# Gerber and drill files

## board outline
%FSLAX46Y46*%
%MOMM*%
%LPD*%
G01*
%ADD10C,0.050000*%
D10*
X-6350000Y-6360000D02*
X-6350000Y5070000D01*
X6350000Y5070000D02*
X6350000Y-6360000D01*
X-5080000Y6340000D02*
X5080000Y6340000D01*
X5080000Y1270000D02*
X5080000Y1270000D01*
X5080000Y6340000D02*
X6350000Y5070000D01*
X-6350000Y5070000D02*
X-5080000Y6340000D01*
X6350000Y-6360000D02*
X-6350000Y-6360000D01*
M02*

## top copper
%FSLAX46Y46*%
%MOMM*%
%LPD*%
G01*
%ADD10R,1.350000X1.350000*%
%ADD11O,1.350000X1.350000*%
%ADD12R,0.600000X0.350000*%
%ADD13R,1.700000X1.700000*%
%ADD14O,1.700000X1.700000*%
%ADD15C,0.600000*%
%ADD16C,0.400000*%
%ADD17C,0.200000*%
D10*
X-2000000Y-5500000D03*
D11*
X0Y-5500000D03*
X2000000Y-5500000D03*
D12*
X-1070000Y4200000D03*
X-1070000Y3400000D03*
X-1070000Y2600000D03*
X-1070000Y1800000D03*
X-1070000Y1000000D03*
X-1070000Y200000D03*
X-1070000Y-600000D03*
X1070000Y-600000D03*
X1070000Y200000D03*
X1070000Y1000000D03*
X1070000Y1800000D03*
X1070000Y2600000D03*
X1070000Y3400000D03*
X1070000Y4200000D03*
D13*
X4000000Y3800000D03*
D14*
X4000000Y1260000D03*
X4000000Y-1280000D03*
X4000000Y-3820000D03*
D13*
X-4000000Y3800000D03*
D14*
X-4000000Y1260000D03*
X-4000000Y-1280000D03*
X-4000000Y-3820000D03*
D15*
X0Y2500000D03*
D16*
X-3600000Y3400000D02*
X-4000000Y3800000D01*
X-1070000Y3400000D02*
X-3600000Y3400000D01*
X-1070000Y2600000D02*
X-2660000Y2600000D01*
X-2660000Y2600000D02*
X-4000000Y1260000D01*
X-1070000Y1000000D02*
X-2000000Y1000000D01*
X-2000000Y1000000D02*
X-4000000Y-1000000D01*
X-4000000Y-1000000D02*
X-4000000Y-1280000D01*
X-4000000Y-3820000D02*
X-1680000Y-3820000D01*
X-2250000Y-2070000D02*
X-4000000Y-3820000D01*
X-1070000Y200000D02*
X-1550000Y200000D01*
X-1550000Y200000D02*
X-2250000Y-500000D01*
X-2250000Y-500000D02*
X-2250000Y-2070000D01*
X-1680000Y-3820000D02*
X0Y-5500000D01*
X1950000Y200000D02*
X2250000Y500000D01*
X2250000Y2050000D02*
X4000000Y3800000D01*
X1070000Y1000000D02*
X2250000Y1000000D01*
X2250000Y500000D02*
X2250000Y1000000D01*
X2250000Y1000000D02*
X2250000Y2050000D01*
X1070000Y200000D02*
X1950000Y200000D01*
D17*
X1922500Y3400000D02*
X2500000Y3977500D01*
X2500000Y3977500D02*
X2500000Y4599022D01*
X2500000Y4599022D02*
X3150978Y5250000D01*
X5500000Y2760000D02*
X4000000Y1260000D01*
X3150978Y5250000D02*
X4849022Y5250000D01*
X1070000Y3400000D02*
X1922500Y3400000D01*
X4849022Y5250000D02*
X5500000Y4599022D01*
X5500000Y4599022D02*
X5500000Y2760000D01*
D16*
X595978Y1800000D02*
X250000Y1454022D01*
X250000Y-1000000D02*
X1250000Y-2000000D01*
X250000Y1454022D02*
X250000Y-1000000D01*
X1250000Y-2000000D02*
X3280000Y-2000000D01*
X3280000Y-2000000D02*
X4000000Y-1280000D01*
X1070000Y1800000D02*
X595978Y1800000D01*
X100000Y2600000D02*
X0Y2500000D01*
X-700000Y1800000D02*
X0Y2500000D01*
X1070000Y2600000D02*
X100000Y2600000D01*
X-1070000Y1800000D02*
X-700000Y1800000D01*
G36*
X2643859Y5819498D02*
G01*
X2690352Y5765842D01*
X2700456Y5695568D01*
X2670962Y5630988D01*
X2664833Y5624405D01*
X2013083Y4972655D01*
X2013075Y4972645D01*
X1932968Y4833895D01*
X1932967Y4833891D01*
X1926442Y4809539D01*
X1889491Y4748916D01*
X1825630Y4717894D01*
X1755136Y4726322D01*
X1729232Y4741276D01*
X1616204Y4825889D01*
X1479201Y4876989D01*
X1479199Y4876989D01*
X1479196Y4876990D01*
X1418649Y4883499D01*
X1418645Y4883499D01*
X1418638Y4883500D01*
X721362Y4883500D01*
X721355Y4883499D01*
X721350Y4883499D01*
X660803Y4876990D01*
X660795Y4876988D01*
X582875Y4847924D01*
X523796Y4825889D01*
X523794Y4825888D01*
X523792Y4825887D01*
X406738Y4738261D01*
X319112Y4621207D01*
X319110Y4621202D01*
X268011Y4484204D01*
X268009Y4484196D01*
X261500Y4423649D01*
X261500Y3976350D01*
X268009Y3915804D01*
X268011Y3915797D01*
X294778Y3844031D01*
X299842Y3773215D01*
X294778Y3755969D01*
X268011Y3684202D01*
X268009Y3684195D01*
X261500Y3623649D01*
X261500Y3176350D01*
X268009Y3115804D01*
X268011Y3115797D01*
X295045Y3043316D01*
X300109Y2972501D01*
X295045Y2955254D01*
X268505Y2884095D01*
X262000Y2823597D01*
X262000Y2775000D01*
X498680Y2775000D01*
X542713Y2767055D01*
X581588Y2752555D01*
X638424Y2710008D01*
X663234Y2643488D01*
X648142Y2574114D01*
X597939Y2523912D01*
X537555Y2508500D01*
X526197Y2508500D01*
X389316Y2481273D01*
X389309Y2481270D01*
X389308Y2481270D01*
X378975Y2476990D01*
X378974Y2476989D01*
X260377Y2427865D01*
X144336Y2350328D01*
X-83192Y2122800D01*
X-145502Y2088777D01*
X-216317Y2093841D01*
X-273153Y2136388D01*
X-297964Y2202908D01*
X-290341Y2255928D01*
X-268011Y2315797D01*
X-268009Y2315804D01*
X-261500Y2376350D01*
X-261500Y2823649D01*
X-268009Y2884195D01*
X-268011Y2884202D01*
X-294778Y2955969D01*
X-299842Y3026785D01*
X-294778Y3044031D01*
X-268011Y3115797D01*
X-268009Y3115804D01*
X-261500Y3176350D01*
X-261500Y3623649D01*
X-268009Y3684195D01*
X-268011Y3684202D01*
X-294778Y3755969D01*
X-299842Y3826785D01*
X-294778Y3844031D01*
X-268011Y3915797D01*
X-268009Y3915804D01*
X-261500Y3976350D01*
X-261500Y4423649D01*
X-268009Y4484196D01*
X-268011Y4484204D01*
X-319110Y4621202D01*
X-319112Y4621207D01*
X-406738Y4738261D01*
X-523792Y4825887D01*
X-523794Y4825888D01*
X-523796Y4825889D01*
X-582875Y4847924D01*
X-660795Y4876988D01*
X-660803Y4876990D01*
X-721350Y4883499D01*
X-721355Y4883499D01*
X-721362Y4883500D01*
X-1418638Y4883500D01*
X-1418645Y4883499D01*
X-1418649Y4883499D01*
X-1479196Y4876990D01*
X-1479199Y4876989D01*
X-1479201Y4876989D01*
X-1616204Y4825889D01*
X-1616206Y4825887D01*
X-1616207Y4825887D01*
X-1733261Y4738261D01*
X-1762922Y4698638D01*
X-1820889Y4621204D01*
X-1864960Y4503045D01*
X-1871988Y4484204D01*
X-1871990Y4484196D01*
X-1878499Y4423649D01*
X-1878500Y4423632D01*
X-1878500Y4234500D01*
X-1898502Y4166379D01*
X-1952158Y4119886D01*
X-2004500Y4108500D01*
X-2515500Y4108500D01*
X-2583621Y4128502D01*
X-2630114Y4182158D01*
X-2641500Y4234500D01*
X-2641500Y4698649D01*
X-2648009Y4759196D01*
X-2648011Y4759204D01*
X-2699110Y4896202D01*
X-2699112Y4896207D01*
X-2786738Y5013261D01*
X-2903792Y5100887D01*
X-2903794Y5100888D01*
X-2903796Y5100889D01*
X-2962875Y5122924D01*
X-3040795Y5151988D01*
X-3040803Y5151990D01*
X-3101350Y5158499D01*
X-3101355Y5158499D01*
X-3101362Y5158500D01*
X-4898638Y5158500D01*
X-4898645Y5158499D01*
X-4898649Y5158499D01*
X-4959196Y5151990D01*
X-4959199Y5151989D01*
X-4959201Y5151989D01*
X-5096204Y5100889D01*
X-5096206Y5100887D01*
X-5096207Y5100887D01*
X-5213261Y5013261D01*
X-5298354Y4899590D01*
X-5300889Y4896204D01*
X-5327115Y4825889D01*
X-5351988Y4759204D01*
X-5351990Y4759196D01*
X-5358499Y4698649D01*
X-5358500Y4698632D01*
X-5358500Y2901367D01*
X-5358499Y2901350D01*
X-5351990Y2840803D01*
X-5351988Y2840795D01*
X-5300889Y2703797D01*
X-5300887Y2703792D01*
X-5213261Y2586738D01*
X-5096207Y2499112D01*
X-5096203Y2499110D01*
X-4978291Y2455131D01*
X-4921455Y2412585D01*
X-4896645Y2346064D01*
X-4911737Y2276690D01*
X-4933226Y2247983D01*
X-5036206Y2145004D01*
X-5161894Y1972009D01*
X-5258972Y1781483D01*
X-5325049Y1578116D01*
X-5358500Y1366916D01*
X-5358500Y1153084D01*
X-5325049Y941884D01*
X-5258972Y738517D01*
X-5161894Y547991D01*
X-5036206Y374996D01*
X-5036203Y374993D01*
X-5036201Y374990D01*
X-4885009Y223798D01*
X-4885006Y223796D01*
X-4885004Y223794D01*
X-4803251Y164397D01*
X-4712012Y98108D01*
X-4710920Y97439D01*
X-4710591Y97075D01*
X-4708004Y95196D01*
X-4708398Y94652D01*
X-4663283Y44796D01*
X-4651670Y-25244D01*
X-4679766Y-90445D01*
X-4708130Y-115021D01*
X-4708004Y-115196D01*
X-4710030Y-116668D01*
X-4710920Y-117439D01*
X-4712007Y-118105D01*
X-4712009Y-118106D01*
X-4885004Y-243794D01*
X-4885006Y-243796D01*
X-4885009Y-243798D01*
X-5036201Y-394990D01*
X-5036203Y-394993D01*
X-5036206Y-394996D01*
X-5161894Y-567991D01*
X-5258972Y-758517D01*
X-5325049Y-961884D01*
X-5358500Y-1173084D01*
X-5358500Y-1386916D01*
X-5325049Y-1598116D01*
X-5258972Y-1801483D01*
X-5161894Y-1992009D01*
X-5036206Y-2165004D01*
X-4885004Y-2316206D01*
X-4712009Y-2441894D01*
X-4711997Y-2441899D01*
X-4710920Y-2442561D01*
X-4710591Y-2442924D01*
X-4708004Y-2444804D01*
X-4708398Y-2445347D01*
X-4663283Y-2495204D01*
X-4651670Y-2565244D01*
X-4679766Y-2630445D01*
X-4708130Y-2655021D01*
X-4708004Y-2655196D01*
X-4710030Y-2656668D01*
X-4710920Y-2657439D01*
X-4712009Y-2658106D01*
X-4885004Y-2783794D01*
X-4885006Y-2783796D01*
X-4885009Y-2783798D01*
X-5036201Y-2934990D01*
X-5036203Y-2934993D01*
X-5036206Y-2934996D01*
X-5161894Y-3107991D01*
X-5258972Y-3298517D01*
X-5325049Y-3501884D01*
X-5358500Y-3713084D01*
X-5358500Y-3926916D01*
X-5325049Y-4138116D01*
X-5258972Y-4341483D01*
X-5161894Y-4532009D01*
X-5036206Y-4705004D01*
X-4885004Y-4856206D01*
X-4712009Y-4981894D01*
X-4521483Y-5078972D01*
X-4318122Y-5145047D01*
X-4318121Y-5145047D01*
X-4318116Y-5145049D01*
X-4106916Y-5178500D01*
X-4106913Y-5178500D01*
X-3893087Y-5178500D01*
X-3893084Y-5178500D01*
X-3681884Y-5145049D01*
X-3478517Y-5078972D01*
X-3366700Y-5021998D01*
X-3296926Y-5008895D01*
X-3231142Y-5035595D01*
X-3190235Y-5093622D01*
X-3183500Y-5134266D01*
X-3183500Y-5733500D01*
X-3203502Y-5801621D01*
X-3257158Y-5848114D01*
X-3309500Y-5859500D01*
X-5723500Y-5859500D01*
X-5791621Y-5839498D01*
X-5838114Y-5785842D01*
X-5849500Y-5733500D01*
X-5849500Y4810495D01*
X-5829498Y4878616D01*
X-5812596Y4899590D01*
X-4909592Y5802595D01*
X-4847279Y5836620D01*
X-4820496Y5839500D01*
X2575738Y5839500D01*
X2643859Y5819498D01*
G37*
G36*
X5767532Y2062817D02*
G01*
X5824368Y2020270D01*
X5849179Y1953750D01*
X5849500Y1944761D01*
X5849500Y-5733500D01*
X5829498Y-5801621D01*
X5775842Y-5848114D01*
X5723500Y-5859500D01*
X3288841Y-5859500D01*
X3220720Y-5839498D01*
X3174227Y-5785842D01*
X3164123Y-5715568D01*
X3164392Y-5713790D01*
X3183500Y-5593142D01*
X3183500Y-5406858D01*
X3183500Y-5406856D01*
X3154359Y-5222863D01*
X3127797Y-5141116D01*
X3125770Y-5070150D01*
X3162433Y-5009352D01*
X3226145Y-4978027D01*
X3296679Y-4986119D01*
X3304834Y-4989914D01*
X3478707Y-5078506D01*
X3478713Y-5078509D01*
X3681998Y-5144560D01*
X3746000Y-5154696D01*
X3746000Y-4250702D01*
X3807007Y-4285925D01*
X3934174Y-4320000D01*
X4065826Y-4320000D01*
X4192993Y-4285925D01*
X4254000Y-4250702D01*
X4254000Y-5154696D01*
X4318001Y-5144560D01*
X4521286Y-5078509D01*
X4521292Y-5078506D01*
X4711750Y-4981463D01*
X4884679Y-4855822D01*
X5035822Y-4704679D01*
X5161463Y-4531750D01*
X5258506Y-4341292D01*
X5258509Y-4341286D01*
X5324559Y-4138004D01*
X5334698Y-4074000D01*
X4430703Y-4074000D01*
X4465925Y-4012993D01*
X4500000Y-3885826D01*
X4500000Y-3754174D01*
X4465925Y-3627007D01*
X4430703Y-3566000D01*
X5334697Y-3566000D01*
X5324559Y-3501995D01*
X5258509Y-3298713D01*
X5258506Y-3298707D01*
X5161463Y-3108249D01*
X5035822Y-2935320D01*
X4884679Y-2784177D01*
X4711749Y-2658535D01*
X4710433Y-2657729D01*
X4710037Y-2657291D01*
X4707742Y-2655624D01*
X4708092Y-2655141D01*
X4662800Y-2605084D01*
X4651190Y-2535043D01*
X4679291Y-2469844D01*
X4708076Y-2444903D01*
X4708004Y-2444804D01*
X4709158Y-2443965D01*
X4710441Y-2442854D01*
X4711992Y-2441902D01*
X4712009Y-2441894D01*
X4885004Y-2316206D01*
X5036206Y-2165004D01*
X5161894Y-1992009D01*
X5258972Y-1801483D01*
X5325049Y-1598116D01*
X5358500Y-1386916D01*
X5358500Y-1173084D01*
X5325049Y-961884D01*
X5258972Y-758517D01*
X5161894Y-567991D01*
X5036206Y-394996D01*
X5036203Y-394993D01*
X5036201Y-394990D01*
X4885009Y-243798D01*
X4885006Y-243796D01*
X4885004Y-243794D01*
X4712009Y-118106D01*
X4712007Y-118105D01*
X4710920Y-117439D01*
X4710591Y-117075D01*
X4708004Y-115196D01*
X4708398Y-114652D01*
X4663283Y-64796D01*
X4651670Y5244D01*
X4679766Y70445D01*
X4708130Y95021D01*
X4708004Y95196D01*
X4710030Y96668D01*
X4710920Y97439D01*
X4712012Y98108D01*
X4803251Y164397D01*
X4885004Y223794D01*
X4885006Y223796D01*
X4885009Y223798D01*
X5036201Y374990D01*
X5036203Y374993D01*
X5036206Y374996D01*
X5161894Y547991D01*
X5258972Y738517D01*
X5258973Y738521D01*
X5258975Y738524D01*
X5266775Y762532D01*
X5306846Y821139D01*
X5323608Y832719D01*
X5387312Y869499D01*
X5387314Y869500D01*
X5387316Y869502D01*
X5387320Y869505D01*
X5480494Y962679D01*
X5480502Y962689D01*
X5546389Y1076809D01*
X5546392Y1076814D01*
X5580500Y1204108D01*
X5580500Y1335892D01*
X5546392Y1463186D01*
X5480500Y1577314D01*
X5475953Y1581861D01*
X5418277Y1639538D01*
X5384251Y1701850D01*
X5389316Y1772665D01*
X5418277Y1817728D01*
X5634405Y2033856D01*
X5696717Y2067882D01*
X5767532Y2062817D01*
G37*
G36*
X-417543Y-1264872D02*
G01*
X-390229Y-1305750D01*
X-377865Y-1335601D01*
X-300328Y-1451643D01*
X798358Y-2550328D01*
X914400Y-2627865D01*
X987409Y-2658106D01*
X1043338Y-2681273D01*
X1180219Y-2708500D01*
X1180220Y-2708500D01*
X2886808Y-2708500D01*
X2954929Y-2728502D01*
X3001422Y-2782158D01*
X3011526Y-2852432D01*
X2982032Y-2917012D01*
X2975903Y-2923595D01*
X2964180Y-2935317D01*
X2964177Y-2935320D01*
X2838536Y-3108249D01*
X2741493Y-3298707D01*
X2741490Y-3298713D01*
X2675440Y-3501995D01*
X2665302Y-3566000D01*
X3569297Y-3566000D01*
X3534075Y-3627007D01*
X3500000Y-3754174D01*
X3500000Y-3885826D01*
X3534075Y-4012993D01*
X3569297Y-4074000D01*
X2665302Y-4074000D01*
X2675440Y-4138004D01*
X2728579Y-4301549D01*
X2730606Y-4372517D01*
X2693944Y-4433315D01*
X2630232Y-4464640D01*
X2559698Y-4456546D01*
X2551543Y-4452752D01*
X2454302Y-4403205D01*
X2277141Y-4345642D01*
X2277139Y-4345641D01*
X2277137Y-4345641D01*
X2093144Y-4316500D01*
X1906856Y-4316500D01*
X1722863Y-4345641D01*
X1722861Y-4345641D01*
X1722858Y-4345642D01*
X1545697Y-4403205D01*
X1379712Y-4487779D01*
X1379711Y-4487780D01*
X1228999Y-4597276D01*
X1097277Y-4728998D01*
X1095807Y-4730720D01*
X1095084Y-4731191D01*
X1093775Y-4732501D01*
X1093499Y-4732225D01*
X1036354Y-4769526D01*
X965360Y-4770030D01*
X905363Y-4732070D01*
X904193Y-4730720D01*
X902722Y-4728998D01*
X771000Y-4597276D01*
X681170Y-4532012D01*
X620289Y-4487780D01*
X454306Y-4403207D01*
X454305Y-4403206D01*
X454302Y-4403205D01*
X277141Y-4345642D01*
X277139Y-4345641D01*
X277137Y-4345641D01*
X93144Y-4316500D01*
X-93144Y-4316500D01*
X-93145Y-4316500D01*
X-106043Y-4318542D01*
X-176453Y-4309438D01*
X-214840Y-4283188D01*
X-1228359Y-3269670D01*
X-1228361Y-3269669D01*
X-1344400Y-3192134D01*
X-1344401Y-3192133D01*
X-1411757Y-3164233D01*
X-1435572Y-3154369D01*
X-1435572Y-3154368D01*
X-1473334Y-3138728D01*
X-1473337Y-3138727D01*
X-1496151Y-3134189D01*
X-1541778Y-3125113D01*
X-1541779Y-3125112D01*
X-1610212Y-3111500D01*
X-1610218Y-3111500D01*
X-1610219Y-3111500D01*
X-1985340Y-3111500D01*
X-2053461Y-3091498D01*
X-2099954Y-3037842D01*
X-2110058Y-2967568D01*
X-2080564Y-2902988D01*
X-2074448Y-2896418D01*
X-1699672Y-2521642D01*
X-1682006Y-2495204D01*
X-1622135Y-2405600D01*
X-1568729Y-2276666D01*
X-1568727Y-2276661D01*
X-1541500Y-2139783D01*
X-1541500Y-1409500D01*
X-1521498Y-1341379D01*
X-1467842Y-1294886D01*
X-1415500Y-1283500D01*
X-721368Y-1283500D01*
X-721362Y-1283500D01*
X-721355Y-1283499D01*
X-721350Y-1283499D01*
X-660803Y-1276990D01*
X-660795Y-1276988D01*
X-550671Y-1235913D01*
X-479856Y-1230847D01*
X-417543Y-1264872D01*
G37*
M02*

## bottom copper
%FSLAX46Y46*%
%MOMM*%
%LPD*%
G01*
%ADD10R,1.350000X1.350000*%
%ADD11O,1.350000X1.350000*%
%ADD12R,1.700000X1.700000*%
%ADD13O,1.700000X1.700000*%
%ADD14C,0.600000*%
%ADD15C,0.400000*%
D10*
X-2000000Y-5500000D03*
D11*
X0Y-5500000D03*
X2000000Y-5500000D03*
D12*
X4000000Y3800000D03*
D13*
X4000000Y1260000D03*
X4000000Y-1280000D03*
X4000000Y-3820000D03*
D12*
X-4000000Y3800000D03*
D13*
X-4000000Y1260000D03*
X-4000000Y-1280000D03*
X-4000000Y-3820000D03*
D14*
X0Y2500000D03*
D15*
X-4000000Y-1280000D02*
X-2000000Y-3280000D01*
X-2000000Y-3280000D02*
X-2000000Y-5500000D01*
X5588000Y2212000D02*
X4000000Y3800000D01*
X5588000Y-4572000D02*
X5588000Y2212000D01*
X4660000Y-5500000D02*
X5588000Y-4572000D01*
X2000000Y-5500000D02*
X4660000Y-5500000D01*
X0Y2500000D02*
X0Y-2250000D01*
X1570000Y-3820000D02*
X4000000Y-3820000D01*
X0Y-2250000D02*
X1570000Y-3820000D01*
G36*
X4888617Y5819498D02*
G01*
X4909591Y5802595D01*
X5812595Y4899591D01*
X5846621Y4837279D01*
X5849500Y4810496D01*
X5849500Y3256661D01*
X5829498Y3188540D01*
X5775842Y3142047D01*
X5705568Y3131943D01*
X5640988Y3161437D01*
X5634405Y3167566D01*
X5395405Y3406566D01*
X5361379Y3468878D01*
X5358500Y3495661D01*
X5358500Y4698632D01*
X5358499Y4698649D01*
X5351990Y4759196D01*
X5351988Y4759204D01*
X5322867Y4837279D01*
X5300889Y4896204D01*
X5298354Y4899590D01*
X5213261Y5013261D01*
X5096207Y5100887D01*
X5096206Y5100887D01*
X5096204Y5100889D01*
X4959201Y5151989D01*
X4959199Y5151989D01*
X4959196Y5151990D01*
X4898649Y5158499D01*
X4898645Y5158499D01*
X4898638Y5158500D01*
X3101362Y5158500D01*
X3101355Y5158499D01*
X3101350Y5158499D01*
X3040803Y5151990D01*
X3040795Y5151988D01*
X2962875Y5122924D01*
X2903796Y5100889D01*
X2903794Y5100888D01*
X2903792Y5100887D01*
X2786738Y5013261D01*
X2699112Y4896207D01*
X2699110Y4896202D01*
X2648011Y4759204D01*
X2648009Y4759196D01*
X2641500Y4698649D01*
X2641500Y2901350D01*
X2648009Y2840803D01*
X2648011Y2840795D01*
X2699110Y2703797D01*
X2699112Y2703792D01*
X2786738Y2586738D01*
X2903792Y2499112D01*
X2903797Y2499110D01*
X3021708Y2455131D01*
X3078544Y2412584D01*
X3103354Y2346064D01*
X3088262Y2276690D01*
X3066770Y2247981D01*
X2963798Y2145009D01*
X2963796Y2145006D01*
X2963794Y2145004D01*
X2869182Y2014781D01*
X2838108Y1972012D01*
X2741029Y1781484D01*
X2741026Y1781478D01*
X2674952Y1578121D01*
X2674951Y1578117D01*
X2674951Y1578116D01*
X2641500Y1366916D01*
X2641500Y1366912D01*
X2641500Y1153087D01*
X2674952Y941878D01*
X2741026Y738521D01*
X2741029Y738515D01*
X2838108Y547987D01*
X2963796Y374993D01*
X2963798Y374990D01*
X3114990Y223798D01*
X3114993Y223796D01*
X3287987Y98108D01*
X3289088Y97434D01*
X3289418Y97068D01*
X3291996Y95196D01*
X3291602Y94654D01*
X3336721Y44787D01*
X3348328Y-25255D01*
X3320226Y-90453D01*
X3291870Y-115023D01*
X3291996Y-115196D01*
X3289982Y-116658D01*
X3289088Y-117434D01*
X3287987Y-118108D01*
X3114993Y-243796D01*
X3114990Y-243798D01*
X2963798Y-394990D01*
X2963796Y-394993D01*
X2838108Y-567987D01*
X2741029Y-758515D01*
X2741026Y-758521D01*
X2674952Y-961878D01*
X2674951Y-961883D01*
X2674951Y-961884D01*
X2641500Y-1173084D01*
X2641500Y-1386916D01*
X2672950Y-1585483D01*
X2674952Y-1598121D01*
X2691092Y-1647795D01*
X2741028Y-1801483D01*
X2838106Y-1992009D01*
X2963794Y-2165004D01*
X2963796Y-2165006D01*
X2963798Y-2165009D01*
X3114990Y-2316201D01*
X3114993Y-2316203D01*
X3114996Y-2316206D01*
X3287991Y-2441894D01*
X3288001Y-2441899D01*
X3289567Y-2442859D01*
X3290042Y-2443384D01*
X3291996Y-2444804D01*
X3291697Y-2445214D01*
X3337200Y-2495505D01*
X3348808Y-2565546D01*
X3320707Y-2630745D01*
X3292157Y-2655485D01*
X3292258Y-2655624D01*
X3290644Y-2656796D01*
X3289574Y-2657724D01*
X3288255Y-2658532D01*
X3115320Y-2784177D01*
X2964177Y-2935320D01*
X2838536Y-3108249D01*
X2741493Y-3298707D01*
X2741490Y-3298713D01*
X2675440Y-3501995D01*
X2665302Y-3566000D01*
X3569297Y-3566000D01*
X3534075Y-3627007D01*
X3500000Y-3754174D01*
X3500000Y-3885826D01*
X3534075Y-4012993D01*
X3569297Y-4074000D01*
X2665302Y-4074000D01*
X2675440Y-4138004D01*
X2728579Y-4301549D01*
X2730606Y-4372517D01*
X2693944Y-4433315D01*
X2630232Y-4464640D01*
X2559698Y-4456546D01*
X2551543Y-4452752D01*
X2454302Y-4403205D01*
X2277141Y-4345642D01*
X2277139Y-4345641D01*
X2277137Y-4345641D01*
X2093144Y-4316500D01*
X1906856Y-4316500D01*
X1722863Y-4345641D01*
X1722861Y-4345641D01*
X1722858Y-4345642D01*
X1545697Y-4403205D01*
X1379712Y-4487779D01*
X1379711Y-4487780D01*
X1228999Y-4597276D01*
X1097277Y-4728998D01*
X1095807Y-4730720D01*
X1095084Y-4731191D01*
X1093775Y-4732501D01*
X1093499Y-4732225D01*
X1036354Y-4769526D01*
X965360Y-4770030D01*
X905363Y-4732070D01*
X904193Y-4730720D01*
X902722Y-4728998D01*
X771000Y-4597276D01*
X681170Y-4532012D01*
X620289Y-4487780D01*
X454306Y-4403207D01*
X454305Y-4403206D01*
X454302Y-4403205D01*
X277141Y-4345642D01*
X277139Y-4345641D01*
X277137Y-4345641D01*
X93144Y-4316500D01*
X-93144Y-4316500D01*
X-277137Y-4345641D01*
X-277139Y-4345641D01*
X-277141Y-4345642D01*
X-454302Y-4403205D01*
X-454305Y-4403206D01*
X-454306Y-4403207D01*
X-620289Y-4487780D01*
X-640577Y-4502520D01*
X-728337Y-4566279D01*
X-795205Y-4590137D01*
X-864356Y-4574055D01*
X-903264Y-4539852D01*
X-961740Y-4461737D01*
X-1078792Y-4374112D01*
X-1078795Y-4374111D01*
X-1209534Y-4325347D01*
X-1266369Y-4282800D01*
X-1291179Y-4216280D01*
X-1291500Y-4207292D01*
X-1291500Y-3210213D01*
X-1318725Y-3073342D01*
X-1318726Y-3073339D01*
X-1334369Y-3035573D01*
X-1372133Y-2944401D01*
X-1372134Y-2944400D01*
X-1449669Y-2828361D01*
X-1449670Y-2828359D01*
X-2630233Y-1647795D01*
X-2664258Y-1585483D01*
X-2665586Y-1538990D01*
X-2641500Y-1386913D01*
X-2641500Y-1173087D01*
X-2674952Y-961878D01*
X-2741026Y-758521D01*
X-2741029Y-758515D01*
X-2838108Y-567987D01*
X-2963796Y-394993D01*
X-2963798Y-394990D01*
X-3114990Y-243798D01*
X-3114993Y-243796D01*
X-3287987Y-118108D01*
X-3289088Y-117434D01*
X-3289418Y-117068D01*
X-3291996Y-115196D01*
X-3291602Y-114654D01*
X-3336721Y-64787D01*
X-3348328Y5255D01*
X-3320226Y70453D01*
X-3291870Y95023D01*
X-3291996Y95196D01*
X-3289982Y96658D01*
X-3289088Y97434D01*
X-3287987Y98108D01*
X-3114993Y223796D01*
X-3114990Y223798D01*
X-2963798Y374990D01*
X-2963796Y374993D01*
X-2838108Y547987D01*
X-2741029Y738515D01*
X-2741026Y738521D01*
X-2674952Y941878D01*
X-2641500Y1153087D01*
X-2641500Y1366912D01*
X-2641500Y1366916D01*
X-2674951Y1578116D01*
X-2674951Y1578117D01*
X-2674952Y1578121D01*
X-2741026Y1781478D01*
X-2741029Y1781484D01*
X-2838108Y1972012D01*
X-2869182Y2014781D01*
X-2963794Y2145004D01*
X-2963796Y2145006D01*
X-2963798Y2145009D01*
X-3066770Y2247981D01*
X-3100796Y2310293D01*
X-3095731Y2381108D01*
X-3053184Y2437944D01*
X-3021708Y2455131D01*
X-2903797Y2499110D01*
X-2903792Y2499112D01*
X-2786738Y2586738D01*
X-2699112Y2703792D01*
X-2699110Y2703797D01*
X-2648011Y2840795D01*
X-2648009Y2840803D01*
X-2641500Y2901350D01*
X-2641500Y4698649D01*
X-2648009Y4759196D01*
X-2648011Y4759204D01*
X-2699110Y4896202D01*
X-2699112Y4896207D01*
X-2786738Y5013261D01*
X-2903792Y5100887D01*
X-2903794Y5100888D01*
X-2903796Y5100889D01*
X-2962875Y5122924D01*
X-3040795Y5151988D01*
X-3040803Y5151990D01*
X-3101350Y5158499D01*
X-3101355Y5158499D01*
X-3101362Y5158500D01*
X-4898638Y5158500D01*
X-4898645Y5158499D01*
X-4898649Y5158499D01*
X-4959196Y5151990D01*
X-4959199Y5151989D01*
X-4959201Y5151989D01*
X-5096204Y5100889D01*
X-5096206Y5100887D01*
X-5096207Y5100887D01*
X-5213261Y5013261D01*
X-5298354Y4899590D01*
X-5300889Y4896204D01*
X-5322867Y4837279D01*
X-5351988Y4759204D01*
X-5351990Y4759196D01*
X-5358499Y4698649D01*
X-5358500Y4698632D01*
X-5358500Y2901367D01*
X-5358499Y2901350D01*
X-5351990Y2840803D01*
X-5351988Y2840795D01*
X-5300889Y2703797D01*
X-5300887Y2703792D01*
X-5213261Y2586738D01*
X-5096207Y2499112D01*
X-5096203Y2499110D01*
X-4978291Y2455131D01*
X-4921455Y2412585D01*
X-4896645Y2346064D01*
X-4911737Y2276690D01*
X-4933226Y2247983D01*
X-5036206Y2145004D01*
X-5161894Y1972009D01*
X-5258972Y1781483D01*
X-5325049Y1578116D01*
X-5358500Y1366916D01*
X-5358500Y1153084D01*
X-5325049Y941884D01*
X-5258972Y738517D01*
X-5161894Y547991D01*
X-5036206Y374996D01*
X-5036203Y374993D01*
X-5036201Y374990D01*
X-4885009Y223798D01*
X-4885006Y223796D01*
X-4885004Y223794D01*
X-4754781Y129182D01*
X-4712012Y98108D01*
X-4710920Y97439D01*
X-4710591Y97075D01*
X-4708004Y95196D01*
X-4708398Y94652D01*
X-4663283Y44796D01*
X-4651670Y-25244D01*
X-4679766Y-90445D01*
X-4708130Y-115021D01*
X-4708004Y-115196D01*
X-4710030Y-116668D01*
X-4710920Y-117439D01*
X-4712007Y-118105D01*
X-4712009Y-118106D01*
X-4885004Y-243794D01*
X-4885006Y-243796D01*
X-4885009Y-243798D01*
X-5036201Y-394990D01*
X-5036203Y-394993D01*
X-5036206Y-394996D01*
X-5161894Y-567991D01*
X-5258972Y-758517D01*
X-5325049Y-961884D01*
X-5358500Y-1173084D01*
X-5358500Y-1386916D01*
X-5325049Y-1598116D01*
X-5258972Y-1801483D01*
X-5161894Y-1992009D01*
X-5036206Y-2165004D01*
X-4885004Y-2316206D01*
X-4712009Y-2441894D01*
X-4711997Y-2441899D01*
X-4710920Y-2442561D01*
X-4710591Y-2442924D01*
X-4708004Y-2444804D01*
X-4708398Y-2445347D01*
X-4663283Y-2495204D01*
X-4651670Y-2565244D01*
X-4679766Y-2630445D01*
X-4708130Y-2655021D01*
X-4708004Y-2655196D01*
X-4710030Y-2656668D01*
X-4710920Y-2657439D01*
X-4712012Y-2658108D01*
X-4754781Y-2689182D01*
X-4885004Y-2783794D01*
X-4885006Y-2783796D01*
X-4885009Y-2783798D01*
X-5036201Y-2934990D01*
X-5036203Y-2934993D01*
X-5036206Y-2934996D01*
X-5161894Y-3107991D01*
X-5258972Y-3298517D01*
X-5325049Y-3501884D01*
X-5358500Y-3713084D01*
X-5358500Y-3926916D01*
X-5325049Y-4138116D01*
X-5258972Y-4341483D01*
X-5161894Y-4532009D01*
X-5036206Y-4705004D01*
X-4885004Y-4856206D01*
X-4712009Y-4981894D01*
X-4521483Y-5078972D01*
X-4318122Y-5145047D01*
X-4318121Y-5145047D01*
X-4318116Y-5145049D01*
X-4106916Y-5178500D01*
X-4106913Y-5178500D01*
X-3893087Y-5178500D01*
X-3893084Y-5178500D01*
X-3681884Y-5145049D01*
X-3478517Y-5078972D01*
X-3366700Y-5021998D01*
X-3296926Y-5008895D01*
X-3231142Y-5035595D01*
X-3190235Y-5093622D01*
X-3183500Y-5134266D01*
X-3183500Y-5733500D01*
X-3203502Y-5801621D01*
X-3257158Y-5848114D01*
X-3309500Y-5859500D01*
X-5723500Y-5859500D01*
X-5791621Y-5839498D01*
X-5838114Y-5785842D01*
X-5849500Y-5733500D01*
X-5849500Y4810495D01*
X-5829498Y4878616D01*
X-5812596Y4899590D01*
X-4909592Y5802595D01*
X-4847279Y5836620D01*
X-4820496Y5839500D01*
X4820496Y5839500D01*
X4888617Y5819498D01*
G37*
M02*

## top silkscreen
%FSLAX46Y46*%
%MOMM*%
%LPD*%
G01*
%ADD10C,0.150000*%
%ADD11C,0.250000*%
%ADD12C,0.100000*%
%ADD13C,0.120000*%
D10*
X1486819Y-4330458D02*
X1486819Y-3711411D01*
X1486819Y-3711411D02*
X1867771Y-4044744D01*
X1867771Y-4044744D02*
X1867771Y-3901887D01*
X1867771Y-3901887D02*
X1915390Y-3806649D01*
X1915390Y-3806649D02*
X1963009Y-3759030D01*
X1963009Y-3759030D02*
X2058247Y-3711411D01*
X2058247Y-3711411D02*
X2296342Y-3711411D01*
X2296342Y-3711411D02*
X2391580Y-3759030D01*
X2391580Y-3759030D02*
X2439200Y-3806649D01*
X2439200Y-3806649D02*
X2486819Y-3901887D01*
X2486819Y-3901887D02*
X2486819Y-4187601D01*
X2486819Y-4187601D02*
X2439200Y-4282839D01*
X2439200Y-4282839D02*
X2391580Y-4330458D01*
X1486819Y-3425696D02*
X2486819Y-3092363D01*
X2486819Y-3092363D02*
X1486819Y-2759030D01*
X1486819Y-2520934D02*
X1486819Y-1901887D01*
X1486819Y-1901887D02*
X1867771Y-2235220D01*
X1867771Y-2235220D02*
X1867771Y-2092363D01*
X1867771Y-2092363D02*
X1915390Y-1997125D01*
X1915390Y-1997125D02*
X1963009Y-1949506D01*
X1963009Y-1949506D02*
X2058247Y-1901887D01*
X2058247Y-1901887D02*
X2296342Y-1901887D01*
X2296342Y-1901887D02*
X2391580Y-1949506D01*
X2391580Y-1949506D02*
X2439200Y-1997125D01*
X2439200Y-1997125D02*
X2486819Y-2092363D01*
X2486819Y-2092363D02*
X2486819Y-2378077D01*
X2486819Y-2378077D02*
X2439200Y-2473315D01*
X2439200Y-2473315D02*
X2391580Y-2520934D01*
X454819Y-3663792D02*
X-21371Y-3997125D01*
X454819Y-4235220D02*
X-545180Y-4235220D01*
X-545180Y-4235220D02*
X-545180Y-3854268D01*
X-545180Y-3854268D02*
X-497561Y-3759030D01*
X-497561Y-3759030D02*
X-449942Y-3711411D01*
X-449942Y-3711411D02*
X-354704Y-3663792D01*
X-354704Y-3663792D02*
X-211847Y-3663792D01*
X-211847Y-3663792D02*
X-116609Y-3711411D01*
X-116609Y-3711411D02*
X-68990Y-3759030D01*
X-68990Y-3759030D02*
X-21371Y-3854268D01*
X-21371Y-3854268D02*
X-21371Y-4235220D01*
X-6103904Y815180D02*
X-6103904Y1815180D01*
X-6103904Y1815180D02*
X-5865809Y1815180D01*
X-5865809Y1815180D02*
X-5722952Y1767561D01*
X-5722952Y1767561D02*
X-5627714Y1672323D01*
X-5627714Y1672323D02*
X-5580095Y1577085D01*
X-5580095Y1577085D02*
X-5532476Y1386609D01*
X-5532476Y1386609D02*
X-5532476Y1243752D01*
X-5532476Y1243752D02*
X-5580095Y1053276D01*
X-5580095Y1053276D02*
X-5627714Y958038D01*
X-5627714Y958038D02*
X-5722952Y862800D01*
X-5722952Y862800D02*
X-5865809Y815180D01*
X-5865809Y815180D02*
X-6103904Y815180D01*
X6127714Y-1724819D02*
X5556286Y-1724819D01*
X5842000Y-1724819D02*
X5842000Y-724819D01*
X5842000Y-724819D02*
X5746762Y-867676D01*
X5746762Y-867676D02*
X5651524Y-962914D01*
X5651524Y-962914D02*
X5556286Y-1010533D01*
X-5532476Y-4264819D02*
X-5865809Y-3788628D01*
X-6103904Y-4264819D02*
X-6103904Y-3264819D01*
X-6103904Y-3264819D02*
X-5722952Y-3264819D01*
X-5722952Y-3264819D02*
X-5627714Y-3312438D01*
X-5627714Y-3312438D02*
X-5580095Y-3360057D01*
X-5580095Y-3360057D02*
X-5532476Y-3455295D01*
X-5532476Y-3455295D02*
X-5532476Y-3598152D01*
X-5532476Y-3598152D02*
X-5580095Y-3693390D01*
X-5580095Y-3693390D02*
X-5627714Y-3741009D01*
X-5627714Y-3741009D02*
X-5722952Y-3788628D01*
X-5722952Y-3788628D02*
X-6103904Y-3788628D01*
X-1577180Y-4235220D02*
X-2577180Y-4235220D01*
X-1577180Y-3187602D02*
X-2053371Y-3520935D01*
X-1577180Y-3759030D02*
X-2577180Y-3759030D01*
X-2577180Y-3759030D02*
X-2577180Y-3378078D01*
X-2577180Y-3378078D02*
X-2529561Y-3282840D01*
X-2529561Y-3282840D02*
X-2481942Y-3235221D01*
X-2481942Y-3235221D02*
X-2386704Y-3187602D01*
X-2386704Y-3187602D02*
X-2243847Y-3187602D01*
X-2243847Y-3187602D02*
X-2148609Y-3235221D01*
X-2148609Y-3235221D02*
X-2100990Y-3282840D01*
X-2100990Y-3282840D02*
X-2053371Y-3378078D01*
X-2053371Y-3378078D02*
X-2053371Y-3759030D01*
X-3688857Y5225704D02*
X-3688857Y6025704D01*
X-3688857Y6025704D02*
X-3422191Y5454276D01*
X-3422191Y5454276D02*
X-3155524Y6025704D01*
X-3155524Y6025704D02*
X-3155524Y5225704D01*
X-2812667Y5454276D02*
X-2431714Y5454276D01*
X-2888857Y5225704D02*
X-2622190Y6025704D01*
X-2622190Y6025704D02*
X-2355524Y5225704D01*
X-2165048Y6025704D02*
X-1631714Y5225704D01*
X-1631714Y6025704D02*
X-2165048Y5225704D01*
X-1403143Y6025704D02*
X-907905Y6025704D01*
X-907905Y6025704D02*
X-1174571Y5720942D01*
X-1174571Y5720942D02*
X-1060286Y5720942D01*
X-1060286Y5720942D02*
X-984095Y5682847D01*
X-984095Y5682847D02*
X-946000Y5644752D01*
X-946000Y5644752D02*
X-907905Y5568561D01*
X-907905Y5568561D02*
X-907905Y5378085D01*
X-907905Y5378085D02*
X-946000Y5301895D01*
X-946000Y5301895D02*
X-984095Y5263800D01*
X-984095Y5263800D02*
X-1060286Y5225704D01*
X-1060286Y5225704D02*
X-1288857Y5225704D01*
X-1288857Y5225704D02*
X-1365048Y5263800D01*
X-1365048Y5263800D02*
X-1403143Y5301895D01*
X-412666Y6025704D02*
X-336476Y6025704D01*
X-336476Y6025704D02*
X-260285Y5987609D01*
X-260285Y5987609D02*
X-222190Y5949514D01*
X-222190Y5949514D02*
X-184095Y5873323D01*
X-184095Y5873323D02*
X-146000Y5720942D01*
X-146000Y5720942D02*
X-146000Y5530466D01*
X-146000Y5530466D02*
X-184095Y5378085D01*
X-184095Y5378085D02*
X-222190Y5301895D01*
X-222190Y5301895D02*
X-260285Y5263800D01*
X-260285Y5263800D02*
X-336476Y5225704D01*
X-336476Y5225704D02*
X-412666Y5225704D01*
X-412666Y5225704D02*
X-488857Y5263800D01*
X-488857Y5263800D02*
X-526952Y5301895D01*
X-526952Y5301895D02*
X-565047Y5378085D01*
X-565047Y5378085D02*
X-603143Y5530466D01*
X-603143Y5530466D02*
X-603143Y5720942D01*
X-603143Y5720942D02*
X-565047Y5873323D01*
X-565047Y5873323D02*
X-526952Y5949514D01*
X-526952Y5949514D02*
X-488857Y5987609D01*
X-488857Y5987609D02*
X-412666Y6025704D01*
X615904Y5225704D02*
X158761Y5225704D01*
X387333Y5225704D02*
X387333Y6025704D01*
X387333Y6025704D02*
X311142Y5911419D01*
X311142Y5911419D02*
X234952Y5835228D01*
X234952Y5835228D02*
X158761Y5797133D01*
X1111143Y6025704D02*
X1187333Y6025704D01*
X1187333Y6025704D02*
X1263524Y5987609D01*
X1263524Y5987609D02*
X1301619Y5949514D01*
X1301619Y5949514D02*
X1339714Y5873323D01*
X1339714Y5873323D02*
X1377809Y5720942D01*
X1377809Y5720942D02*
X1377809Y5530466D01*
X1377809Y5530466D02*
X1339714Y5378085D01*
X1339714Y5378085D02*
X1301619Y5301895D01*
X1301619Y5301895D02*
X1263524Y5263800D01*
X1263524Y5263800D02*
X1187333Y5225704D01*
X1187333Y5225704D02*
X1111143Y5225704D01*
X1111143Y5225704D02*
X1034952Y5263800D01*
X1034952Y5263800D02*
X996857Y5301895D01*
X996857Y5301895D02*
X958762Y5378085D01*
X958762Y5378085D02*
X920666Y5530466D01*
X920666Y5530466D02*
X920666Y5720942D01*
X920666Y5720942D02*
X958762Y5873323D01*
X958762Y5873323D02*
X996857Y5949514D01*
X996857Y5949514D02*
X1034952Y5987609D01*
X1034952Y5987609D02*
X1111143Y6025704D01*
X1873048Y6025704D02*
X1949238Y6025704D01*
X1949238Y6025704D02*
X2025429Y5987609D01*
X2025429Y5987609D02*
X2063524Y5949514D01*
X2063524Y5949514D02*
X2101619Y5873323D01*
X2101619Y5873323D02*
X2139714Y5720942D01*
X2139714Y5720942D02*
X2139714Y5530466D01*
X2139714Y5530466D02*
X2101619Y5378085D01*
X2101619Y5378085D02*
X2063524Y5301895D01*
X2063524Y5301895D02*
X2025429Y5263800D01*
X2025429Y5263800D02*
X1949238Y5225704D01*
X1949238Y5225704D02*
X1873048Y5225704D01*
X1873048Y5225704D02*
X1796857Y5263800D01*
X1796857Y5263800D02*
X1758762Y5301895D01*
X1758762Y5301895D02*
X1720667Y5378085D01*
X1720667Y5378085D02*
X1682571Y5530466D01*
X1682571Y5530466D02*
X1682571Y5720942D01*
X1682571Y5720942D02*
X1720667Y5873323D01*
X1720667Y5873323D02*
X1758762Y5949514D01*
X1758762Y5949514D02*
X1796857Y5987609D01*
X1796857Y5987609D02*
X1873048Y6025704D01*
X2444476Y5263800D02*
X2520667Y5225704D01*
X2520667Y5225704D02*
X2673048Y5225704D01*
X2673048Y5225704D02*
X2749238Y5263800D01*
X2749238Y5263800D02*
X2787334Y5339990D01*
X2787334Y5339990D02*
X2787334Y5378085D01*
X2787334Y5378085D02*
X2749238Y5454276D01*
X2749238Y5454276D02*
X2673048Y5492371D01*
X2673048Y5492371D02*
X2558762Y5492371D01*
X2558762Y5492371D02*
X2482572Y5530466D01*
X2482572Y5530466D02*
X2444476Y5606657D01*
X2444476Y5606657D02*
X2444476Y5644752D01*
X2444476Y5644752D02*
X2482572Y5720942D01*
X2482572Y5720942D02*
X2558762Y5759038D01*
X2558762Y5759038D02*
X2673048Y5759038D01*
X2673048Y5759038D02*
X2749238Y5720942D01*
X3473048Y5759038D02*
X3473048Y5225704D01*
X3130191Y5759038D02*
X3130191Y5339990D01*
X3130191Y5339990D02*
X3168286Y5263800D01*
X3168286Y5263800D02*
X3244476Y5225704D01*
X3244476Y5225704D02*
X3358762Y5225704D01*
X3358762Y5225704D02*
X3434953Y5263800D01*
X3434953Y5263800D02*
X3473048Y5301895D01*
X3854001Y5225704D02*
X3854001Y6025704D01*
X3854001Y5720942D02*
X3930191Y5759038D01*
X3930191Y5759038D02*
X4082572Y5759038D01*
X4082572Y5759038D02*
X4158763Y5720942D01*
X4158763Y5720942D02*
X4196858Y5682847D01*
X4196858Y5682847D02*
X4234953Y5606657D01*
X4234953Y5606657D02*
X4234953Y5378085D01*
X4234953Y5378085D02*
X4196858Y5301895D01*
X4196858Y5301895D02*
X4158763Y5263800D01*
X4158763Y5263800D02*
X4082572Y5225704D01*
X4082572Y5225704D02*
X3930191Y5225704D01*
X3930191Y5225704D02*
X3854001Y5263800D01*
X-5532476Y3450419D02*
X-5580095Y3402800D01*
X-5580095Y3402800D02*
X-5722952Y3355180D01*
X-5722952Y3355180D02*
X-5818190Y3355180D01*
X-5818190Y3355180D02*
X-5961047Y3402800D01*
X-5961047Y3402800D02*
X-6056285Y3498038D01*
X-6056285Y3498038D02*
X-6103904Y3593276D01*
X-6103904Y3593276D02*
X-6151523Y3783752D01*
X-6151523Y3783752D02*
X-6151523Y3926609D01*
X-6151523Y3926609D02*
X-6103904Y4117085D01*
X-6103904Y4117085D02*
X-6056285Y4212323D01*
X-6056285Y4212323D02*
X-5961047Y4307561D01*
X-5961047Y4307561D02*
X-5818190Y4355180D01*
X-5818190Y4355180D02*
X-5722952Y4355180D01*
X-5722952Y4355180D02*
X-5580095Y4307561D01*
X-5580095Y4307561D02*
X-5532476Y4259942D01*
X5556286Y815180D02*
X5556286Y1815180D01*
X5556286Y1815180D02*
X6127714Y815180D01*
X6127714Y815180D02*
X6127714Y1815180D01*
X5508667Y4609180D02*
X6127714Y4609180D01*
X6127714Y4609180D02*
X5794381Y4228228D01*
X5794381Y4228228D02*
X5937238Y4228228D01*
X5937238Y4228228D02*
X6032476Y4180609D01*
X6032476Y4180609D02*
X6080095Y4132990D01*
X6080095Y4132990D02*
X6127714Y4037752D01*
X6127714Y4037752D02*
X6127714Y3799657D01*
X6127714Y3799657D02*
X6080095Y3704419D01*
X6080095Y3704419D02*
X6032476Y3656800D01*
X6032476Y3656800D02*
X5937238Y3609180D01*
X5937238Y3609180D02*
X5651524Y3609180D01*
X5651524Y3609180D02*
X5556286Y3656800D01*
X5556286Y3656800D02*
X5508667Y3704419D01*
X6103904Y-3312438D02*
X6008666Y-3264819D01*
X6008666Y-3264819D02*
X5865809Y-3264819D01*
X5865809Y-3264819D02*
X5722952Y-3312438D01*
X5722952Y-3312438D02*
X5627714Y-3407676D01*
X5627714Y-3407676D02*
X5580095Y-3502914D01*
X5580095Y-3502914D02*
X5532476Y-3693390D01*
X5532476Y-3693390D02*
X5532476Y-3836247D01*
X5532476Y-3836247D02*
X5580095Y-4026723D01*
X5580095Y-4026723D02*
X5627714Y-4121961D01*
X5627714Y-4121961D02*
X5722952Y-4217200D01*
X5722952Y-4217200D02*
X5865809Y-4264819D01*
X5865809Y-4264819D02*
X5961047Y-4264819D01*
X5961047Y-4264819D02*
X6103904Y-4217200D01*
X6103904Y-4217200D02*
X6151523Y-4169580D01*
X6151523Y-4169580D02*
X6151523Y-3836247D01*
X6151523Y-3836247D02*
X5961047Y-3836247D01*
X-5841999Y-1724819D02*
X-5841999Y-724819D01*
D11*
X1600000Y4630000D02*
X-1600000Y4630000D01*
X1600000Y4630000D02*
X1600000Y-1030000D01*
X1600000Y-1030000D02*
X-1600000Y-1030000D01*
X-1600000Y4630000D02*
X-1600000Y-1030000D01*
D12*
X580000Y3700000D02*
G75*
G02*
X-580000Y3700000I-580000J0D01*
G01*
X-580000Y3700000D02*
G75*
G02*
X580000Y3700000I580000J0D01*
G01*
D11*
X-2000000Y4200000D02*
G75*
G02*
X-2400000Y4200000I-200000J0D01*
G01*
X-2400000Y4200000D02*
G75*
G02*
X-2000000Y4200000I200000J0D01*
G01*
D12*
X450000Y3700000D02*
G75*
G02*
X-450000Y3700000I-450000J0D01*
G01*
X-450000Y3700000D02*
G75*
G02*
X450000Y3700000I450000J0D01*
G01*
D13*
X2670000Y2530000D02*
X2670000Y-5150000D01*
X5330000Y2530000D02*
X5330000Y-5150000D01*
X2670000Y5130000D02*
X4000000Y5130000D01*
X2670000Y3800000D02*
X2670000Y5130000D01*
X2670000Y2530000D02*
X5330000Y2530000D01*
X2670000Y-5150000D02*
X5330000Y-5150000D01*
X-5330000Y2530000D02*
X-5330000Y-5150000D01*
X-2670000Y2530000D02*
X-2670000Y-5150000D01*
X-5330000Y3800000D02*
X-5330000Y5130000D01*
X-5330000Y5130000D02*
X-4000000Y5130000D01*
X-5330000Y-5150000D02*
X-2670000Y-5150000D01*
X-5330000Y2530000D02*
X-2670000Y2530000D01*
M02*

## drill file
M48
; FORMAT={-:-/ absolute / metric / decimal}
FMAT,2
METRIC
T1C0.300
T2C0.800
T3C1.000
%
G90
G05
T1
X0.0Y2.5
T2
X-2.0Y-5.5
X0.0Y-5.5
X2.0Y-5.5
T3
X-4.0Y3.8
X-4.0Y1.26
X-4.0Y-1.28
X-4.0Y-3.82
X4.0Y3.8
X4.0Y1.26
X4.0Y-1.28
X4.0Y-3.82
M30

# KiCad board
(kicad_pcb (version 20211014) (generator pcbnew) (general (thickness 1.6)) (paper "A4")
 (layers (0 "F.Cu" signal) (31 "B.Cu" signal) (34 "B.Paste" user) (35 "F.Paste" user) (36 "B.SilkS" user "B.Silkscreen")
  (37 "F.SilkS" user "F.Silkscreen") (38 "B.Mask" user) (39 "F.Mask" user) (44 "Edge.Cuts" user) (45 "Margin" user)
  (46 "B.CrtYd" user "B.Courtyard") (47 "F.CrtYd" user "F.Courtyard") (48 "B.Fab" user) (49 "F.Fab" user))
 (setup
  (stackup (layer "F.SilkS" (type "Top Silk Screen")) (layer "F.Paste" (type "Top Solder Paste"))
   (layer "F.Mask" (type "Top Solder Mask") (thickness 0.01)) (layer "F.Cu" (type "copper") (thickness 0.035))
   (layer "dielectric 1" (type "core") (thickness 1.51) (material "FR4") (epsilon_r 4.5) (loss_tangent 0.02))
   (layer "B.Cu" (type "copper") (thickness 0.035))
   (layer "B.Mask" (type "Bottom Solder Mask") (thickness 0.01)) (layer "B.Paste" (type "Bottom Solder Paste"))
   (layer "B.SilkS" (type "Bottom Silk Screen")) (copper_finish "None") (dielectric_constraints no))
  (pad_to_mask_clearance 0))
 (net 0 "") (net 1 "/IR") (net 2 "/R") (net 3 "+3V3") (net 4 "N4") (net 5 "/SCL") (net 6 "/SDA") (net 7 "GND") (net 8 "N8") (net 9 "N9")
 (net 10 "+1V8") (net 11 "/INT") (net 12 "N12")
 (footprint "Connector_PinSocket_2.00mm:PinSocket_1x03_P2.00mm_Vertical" (layer "F.Cu") (at -2 5.5 90)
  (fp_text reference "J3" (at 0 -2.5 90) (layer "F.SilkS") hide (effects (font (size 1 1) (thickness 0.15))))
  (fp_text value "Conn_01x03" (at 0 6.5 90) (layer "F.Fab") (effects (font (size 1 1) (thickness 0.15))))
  (pad "1" thru_hole rect (at 0 0 90) (size 1.35 1.35) (drill 0.8) (layers *.Cu *.Mask) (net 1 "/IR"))
  (pad "2" thru_hole oval (at 0 2 90) (size 1.35 1.35) (drill 0.8) (layers *.Cu *.Mask) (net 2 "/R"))
  (pad "3" thru_hole oval (at 0 4 90) (size 1.35 1.35) (drill 0.8) (layers *.Cu *.Mask) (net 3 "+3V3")))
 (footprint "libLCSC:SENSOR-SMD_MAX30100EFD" (layer "F.Cu") (at 0 -1.8 -90)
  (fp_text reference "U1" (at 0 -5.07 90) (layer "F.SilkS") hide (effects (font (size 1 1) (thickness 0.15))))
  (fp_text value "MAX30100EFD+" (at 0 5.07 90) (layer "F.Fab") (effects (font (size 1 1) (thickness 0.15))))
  (fp_line (start -2.83 -1.6) (end -2.83 1.6) (layer "F.SilkS") (width 0.25))
  (fp_line (start -2.83 -1.6) (end 2.83 -1.6) (layer "F.SilkS") (width 0.25))
  (fp_line (start 2.83 -1.6) (end 2.83 1.6) (layer "F.SilkS") (width 0.25))
  (fp_line (start -2.83 1.6) (end 2.83 1.6) (layer "F.SilkS") (width 0.25))
  (fp_circle (center -1.9 0) (end -1.32 0) (layer "F.SilkS") (width 0.1) (fill none))
  (fp_circle (center -2.4 2.2) (end -2.2 2.2) (layer "F.SilkS") (width 0.25) (fill none))
  (fp_circle (center -1.9 0) (end -1.45 0) (layer "F.SilkS") (width 0.1) (fill none))
  (pad "1" smd rect locked (at -2.4 1.07 90) (size 0.35 0.6) (layers "F.Cu" "F.Paste" "F.Mask") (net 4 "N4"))
  (pad "2" smd rect locked (at -1.6 1.07 90) (size 0.35 0.6) (layers "F.Cu" "F.Paste" "F.Mask") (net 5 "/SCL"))
  (pad "3" smd rect locked (at -0.8 1.07 90) (size 0.35 0.6) (layers "F.Cu" "F.Paste" "F.Mask") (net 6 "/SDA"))
  (pad "4" smd rect locked (at 0 1.07 90) (size 0.35 0.6) (layers "F.Cu" "F.Paste" "F.Mask") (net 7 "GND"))
  (pad "5" smd rect locked (at 0.8 1.07 90) (size 0.35 0.6) (layers "F.Cu" "F.Paste" "F.Mask") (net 1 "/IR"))
  (pad "6" smd rect locked (at 1.6 1.07 90) (size 0.35 0.6) (layers "F.Cu" "F.Paste" "F.Mask") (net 2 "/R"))
  (pad "7" smd rect locked (at 2.4 1.07 90) (size 0.35 0.6) (layers "F.Cu" "F.Paste" "F.Mask") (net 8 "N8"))
  (pad "8" smd rect locked (at 2.4 -1.07 90) (size 0.35 0.6) (layers "F.Cu" "F.Paste" "F.Mask") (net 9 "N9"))
  (pad "9" smd rect locked (at 1.6 -1.07 90) (size 0.35 0.6) (layers "F.Cu" "F.Paste" "F.Mask") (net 3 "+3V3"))
  (pad "10" smd rect locked (at 0.8 -1.07 90) (size 0.35 0.6) (layers "F.Cu" "F.Paste" "F.Mask") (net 3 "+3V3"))
  (pad "11" smd rect locked (at 0 -1.07 90) (size 0.35 0.6) (layers "F.Cu" "F.Paste" "F.Mask") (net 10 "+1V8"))
  (pad "12" smd rect locked (at -0.8 -1.07 90) (size 0.35 0.6) (layers "F.Cu" "F.Paste" "F.Mask") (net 7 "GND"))
  (pad "13" smd rect locked (at -1.6 -1.07 90) (size 0.35 0.6) (layers "F.Cu" "F.Paste" "F.Mask") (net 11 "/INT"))
  (pad "14" smd rect locked (at -2.4 -1.07 90) (size 0.35 0.6) (layers "F.Cu" "F.Paste" "F.Mask") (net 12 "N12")))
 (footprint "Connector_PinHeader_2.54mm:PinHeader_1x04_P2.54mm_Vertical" (layer "F.Cu") (at 4 -3.8)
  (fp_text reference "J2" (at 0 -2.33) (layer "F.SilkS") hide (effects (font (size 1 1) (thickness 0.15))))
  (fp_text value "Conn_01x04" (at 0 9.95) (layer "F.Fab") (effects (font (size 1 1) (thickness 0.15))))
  (fp_line (start -1.33 1.27) (end -1.33 8.95) (layer "F.SilkS") (width 0.12))
  (fp_line (start 1.33 1.27) (end 1.33 8.95) (layer "F.SilkS") (width 0.12))
  (fp_line (start -1.33 -1.33) (end 0 -1.33) (layer "F.SilkS") (width 0.12))
  (fp_line (start -1.33 0) (end -1.33 -1.33) (layer "F.SilkS") (width 0.12))
  (fp_line (start -1.33 1.27) (end 1.33 1.27) (layer "F.SilkS") (width 0.12))
  (fp_line (start -1.33 8.95) (end 1.33 8.95) (layer "F.SilkS") (width 0.12))
  (pad "1" thru_hole rect locked (at 0 0) (size 1.7 1.7) (drill 1) (layers *.Cu *.Mask) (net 3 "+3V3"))
  (pad "2" thru_hole oval locked (at 0 2.54) (size 1.7 1.7) (drill 1) (layers *.Cu *.Mask) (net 11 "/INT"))
  (pad "3" thru_hole oval locked (at 0 5.08) (size 1.7 1.7) (drill 1) (layers *.Cu *.Mask) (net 10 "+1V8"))
  (pad "4" thru_hole oval locked (at 0 7.62) (size 1.7 1.7) (drill 1) (layers *.Cu *.Mask) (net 7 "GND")))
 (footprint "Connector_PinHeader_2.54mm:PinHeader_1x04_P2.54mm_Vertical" (layer "F.Cu") (at -4 -3.8)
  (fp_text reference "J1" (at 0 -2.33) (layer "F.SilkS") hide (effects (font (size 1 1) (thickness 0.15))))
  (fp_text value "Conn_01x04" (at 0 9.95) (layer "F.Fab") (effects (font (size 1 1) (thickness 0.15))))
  (fp_line (start -1.33 1.27) (end -1.33 8.95) (layer "F.SilkS") (width 0.12))
  (fp_line (start 1.33 1.27) (end 1.33 8.95) (layer "F.SilkS") (width 0.12))
  (fp_line (start -1.33 0) (end -1.33 -1.33) (layer "F.SilkS") (width 0.12))
  (fp_line (start -1.33 -1.33) (end 0 -1.33) (layer "F.SilkS") (width 0.12))
  (fp_line (start -1.33 8.95) (end 1.33 8.95) (layer "F.SilkS") (width 0.12))
  (fp_line (start -1.33 1.27) (end 1.33 1.27) (layer "F.SilkS") (width 0.12))
  (pad "1" thru_hole rect locked (at 0 0) (size 1.7 1.7) (drill 1) (layers *.Cu *.Mask) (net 5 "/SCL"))
  (pad "2" thru_hole oval locked (at 0 2.54) (size 1.7 1.7) (drill 1) (layers *.Cu *.Mask) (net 6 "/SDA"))
  (pad "3" thru_hole oval locked (at 0 5.08) (size 1.7 1.7) (drill 1) (layers *.Cu *.Mask) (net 1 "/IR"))
  (pad "4" thru_hole oval locked (at 0 7.62) (size 1.7 1.7) (drill 1) (layers *.Cu *.Mask) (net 2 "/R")))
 (gr_line (start -6.35 6.36) (end -6.35 -5.07) (layer "Edge.Cuts") (width 0.05))
 (gr_line (start 6.35 -5.07) (end 6.35 6.36) (layer "Edge.Cuts") (width 0.05))
 (gr_line (start -5.08 -6.34) (end 5.08 -6.34) (layer "Edge.Cuts") (width 0.05))
 (gr_line (start 5.08 -1.27) (end 5.08 -1.27) (layer "Edge.Cuts") (width 0.05))
 (gr_line (start 5.08 -6.34) (end 6.35 -5.07) (layer "Edge.Cuts") (width 0.05))
 (gr_line (start -6.35 -5.07) (end -5.08 -6.34) (layer "Edge.Cuts") (width 0.05))
 (gr_line (start 6.35 6.36) (end -6.35 6.36) (layer "Edge.Cuts") (width 0.05))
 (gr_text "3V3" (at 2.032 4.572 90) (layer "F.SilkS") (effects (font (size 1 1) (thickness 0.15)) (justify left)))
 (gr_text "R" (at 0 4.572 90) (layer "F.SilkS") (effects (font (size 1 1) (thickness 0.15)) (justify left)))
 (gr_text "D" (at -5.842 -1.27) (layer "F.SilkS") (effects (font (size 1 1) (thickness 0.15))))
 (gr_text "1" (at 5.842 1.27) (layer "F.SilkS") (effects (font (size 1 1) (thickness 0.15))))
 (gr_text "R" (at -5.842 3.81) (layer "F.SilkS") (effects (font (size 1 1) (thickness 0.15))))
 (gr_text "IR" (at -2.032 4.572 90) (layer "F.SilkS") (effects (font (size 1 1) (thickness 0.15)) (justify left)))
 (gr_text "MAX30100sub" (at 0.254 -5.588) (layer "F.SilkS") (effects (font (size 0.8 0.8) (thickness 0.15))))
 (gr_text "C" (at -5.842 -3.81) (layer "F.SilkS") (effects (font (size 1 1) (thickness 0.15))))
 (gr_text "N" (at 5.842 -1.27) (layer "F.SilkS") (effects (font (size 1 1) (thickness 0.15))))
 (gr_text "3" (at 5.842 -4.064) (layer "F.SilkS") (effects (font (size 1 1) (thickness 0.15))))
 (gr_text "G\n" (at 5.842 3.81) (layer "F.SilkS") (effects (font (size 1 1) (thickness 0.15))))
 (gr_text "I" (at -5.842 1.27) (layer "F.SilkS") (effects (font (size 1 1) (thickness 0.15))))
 (segment (start -3.6 -3.4) (end -4 -3.8) (width 0.4) (layer "F.Cu") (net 5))
 (segment (start -1.07 -3.4) (end -3.6 -3.4) (width 0.4) (layer "F.Cu") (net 5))
 (segment (start -1.07 -2.6) (end -2.66 -2.6) (width 0.4) (layer "F.Cu") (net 6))
 (segment (start -2.66 -2.6) (end -4 -1.26) (width 0.4) (layer "F.Cu") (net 6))
 (segment (start -1.07 -1) (end -2 -1) (width 0.4) (layer "F.Cu") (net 1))
 (segment (start -2 -1) (end -4 1) (width 0.4) (layer "F.Cu") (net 1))
 (segment (start -4 1) (end -4 1.28) (width 0.4) (layer "F.Cu") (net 1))
 (segment (start -4 1.28) (end -2 3.28) (width 0.4) (layer "B.Cu") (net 1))
 (segment (start -2 3.28) (end -2 5.5) (width 0.4) (layer "B.Cu") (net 1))
 (segment (start -4 3.82) (end -1.68 3.82) (width 0.4) (layer "F.Cu") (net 2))
 (segment (start -2.25 2.07) (end -4 3.82) (width 0.4) (layer "F.Cu") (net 2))
 (segment (start -1.07 -0.2) (end -1.55 -0.2) (width 0.4) (layer "F.Cu") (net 2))
 (segment (start -1.55 -0.2) (end -2.25 0.5) (width 0.4) (layer "F.Cu") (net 2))
 (segment (start -2.25 0.5) (end -2.25 2.07) (width 0.4) (layer "F.Cu") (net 2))
 (segment (start -1.68 3.82) (end 0 5.5) (width 0.4) (layer "F.Cu") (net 2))
 (segment (start 1.95 -0.2) (end 2.25 -0.5) (width 0.4) (layer "F.Cu") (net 3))
 (segment (start 2.25 -2.05) (end 4 -3.8) (width 0.4) (layer "F.Cu") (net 3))
 (segment (start 1.07 -1) (end 2.25 -1) (width 0.4) (layer "F.Cu") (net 3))
 (segment (start 2.25 -0.5) (end 2.25 -1) (width 0.4) (layer "F.Cu") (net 3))
 (segment (start 2.25 -1) (end 2.25 -2.05) (width 0.4) (layer "F.Cu") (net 3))
 (segment (start 1.07 -0.2) (end 1.95 -0.2) (width 0.4) (layer "F.Cu") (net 3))
 (segment (start 5.588 -2.212) (end 4 -3.8) (width 0.4) (layer "B.Cu") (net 3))
 (segment (start 5.588 4.572) (end 5.588 -2.212) (width 0.4) (layer "B.Cu") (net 3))
 (segment (start 4.66 5.5) (end 5.588 4.572) (width 0.4) (layer "B.Cu") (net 3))
 (segment (start 2 5.5) (end 4.66 5.5) (width 0.4) (layer "B.Cu") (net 3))
 (segment (start 1.9225 -3.4) (end 2.5 -3.9775) (width 0.2) (layer "F.Cu") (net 11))
 (segment (start 2.5 -3.9775) (end 2.5 -4.599022) (width 0.2) (layer "F.Cu") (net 11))
 (segment (start 2.5 -4.599022) (end 3.150978 -5.25) (width 0.2) (layer "F.Cu") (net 11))
 (segment (start 5.5 -2.76) (end 4 -1.26) (width 0.2) (layer "F.Cu") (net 11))
 (segment (start 3.150978 -5.25) (end 4.849022 -5.25) (width 0.2) (layer "F.Cu") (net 11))
 (segment (start 1.07 -3.4) (end 1.9225 -3.4) (width 0.2) (layer "F.Cu") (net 11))
 (segment (start 4.849022 -5.25) (end 5.5 -4.599022) (width 0.2) (layer "F.Cu") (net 11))
 (segment (start 5.5 -4.599022) (end 5.5 -2.76) (width 0.2) (layer "F.Cu") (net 11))
 (segment (start 0.595978 -1.8) (end 0.25 -1.454022) (width 0.4) (layer "F.Cu") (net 10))
 (segment (start 0.25 1) (end 1.25 2) (width 0.4) (layer "F.Cu") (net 10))
 (segment (start 0.25 -1.454022) (end 0.25 1) (width 0.4) (layer "F.Cu") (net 10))
 (segment (start 1.25 2) (end 3.28 2) (width 0.4) (layer "F.Cu") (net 10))
 (segment (start 3.28 2) (end 4 1.28) (width 0.4) (layer "F.Cu") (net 10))
 (segment (start 1.07 -1.8) (end 0.595978 -1.8) (width 0.4) (layer "F.Cu") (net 10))
 (segment (start 0.1 -2.6) (end 0 -2.5) (width 0.4) (layer "F.Cu") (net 7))
 (segment (start -0.7 -1.8) (end 0 -2.5) (width 0.4) (layer "F.Cu") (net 7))
 (segment (start 1.07 -2.6) (end 0.1 -2.6) (width 0.4) (layer "F.Cu") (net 7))
 (segment (start -1.07 -1.8) (end -0.7 -1.8) (width 0.4) (layer "F.Cu") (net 7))
 (via (at 0 -2.5) (size 0.6) (drill 0.3) (layers "F.Cu" "B.Cu") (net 7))
 (segment (start 0 -2.5) (end 0 2.25) (width 0.4) (layer "B.Cu") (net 7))
 (segment (start 1.57 3.82) (end 4 3.82) (width 0.4) (layer "B.Cu") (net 7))
 (segment (start 0 2.25) (end 1.57 3.82) (width 0.4) (layer "B.Cu") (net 7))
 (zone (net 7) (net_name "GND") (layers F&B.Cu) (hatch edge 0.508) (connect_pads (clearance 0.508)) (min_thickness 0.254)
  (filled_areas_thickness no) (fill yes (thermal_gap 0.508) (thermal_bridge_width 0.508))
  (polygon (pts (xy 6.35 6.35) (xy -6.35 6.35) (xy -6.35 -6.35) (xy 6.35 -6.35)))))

